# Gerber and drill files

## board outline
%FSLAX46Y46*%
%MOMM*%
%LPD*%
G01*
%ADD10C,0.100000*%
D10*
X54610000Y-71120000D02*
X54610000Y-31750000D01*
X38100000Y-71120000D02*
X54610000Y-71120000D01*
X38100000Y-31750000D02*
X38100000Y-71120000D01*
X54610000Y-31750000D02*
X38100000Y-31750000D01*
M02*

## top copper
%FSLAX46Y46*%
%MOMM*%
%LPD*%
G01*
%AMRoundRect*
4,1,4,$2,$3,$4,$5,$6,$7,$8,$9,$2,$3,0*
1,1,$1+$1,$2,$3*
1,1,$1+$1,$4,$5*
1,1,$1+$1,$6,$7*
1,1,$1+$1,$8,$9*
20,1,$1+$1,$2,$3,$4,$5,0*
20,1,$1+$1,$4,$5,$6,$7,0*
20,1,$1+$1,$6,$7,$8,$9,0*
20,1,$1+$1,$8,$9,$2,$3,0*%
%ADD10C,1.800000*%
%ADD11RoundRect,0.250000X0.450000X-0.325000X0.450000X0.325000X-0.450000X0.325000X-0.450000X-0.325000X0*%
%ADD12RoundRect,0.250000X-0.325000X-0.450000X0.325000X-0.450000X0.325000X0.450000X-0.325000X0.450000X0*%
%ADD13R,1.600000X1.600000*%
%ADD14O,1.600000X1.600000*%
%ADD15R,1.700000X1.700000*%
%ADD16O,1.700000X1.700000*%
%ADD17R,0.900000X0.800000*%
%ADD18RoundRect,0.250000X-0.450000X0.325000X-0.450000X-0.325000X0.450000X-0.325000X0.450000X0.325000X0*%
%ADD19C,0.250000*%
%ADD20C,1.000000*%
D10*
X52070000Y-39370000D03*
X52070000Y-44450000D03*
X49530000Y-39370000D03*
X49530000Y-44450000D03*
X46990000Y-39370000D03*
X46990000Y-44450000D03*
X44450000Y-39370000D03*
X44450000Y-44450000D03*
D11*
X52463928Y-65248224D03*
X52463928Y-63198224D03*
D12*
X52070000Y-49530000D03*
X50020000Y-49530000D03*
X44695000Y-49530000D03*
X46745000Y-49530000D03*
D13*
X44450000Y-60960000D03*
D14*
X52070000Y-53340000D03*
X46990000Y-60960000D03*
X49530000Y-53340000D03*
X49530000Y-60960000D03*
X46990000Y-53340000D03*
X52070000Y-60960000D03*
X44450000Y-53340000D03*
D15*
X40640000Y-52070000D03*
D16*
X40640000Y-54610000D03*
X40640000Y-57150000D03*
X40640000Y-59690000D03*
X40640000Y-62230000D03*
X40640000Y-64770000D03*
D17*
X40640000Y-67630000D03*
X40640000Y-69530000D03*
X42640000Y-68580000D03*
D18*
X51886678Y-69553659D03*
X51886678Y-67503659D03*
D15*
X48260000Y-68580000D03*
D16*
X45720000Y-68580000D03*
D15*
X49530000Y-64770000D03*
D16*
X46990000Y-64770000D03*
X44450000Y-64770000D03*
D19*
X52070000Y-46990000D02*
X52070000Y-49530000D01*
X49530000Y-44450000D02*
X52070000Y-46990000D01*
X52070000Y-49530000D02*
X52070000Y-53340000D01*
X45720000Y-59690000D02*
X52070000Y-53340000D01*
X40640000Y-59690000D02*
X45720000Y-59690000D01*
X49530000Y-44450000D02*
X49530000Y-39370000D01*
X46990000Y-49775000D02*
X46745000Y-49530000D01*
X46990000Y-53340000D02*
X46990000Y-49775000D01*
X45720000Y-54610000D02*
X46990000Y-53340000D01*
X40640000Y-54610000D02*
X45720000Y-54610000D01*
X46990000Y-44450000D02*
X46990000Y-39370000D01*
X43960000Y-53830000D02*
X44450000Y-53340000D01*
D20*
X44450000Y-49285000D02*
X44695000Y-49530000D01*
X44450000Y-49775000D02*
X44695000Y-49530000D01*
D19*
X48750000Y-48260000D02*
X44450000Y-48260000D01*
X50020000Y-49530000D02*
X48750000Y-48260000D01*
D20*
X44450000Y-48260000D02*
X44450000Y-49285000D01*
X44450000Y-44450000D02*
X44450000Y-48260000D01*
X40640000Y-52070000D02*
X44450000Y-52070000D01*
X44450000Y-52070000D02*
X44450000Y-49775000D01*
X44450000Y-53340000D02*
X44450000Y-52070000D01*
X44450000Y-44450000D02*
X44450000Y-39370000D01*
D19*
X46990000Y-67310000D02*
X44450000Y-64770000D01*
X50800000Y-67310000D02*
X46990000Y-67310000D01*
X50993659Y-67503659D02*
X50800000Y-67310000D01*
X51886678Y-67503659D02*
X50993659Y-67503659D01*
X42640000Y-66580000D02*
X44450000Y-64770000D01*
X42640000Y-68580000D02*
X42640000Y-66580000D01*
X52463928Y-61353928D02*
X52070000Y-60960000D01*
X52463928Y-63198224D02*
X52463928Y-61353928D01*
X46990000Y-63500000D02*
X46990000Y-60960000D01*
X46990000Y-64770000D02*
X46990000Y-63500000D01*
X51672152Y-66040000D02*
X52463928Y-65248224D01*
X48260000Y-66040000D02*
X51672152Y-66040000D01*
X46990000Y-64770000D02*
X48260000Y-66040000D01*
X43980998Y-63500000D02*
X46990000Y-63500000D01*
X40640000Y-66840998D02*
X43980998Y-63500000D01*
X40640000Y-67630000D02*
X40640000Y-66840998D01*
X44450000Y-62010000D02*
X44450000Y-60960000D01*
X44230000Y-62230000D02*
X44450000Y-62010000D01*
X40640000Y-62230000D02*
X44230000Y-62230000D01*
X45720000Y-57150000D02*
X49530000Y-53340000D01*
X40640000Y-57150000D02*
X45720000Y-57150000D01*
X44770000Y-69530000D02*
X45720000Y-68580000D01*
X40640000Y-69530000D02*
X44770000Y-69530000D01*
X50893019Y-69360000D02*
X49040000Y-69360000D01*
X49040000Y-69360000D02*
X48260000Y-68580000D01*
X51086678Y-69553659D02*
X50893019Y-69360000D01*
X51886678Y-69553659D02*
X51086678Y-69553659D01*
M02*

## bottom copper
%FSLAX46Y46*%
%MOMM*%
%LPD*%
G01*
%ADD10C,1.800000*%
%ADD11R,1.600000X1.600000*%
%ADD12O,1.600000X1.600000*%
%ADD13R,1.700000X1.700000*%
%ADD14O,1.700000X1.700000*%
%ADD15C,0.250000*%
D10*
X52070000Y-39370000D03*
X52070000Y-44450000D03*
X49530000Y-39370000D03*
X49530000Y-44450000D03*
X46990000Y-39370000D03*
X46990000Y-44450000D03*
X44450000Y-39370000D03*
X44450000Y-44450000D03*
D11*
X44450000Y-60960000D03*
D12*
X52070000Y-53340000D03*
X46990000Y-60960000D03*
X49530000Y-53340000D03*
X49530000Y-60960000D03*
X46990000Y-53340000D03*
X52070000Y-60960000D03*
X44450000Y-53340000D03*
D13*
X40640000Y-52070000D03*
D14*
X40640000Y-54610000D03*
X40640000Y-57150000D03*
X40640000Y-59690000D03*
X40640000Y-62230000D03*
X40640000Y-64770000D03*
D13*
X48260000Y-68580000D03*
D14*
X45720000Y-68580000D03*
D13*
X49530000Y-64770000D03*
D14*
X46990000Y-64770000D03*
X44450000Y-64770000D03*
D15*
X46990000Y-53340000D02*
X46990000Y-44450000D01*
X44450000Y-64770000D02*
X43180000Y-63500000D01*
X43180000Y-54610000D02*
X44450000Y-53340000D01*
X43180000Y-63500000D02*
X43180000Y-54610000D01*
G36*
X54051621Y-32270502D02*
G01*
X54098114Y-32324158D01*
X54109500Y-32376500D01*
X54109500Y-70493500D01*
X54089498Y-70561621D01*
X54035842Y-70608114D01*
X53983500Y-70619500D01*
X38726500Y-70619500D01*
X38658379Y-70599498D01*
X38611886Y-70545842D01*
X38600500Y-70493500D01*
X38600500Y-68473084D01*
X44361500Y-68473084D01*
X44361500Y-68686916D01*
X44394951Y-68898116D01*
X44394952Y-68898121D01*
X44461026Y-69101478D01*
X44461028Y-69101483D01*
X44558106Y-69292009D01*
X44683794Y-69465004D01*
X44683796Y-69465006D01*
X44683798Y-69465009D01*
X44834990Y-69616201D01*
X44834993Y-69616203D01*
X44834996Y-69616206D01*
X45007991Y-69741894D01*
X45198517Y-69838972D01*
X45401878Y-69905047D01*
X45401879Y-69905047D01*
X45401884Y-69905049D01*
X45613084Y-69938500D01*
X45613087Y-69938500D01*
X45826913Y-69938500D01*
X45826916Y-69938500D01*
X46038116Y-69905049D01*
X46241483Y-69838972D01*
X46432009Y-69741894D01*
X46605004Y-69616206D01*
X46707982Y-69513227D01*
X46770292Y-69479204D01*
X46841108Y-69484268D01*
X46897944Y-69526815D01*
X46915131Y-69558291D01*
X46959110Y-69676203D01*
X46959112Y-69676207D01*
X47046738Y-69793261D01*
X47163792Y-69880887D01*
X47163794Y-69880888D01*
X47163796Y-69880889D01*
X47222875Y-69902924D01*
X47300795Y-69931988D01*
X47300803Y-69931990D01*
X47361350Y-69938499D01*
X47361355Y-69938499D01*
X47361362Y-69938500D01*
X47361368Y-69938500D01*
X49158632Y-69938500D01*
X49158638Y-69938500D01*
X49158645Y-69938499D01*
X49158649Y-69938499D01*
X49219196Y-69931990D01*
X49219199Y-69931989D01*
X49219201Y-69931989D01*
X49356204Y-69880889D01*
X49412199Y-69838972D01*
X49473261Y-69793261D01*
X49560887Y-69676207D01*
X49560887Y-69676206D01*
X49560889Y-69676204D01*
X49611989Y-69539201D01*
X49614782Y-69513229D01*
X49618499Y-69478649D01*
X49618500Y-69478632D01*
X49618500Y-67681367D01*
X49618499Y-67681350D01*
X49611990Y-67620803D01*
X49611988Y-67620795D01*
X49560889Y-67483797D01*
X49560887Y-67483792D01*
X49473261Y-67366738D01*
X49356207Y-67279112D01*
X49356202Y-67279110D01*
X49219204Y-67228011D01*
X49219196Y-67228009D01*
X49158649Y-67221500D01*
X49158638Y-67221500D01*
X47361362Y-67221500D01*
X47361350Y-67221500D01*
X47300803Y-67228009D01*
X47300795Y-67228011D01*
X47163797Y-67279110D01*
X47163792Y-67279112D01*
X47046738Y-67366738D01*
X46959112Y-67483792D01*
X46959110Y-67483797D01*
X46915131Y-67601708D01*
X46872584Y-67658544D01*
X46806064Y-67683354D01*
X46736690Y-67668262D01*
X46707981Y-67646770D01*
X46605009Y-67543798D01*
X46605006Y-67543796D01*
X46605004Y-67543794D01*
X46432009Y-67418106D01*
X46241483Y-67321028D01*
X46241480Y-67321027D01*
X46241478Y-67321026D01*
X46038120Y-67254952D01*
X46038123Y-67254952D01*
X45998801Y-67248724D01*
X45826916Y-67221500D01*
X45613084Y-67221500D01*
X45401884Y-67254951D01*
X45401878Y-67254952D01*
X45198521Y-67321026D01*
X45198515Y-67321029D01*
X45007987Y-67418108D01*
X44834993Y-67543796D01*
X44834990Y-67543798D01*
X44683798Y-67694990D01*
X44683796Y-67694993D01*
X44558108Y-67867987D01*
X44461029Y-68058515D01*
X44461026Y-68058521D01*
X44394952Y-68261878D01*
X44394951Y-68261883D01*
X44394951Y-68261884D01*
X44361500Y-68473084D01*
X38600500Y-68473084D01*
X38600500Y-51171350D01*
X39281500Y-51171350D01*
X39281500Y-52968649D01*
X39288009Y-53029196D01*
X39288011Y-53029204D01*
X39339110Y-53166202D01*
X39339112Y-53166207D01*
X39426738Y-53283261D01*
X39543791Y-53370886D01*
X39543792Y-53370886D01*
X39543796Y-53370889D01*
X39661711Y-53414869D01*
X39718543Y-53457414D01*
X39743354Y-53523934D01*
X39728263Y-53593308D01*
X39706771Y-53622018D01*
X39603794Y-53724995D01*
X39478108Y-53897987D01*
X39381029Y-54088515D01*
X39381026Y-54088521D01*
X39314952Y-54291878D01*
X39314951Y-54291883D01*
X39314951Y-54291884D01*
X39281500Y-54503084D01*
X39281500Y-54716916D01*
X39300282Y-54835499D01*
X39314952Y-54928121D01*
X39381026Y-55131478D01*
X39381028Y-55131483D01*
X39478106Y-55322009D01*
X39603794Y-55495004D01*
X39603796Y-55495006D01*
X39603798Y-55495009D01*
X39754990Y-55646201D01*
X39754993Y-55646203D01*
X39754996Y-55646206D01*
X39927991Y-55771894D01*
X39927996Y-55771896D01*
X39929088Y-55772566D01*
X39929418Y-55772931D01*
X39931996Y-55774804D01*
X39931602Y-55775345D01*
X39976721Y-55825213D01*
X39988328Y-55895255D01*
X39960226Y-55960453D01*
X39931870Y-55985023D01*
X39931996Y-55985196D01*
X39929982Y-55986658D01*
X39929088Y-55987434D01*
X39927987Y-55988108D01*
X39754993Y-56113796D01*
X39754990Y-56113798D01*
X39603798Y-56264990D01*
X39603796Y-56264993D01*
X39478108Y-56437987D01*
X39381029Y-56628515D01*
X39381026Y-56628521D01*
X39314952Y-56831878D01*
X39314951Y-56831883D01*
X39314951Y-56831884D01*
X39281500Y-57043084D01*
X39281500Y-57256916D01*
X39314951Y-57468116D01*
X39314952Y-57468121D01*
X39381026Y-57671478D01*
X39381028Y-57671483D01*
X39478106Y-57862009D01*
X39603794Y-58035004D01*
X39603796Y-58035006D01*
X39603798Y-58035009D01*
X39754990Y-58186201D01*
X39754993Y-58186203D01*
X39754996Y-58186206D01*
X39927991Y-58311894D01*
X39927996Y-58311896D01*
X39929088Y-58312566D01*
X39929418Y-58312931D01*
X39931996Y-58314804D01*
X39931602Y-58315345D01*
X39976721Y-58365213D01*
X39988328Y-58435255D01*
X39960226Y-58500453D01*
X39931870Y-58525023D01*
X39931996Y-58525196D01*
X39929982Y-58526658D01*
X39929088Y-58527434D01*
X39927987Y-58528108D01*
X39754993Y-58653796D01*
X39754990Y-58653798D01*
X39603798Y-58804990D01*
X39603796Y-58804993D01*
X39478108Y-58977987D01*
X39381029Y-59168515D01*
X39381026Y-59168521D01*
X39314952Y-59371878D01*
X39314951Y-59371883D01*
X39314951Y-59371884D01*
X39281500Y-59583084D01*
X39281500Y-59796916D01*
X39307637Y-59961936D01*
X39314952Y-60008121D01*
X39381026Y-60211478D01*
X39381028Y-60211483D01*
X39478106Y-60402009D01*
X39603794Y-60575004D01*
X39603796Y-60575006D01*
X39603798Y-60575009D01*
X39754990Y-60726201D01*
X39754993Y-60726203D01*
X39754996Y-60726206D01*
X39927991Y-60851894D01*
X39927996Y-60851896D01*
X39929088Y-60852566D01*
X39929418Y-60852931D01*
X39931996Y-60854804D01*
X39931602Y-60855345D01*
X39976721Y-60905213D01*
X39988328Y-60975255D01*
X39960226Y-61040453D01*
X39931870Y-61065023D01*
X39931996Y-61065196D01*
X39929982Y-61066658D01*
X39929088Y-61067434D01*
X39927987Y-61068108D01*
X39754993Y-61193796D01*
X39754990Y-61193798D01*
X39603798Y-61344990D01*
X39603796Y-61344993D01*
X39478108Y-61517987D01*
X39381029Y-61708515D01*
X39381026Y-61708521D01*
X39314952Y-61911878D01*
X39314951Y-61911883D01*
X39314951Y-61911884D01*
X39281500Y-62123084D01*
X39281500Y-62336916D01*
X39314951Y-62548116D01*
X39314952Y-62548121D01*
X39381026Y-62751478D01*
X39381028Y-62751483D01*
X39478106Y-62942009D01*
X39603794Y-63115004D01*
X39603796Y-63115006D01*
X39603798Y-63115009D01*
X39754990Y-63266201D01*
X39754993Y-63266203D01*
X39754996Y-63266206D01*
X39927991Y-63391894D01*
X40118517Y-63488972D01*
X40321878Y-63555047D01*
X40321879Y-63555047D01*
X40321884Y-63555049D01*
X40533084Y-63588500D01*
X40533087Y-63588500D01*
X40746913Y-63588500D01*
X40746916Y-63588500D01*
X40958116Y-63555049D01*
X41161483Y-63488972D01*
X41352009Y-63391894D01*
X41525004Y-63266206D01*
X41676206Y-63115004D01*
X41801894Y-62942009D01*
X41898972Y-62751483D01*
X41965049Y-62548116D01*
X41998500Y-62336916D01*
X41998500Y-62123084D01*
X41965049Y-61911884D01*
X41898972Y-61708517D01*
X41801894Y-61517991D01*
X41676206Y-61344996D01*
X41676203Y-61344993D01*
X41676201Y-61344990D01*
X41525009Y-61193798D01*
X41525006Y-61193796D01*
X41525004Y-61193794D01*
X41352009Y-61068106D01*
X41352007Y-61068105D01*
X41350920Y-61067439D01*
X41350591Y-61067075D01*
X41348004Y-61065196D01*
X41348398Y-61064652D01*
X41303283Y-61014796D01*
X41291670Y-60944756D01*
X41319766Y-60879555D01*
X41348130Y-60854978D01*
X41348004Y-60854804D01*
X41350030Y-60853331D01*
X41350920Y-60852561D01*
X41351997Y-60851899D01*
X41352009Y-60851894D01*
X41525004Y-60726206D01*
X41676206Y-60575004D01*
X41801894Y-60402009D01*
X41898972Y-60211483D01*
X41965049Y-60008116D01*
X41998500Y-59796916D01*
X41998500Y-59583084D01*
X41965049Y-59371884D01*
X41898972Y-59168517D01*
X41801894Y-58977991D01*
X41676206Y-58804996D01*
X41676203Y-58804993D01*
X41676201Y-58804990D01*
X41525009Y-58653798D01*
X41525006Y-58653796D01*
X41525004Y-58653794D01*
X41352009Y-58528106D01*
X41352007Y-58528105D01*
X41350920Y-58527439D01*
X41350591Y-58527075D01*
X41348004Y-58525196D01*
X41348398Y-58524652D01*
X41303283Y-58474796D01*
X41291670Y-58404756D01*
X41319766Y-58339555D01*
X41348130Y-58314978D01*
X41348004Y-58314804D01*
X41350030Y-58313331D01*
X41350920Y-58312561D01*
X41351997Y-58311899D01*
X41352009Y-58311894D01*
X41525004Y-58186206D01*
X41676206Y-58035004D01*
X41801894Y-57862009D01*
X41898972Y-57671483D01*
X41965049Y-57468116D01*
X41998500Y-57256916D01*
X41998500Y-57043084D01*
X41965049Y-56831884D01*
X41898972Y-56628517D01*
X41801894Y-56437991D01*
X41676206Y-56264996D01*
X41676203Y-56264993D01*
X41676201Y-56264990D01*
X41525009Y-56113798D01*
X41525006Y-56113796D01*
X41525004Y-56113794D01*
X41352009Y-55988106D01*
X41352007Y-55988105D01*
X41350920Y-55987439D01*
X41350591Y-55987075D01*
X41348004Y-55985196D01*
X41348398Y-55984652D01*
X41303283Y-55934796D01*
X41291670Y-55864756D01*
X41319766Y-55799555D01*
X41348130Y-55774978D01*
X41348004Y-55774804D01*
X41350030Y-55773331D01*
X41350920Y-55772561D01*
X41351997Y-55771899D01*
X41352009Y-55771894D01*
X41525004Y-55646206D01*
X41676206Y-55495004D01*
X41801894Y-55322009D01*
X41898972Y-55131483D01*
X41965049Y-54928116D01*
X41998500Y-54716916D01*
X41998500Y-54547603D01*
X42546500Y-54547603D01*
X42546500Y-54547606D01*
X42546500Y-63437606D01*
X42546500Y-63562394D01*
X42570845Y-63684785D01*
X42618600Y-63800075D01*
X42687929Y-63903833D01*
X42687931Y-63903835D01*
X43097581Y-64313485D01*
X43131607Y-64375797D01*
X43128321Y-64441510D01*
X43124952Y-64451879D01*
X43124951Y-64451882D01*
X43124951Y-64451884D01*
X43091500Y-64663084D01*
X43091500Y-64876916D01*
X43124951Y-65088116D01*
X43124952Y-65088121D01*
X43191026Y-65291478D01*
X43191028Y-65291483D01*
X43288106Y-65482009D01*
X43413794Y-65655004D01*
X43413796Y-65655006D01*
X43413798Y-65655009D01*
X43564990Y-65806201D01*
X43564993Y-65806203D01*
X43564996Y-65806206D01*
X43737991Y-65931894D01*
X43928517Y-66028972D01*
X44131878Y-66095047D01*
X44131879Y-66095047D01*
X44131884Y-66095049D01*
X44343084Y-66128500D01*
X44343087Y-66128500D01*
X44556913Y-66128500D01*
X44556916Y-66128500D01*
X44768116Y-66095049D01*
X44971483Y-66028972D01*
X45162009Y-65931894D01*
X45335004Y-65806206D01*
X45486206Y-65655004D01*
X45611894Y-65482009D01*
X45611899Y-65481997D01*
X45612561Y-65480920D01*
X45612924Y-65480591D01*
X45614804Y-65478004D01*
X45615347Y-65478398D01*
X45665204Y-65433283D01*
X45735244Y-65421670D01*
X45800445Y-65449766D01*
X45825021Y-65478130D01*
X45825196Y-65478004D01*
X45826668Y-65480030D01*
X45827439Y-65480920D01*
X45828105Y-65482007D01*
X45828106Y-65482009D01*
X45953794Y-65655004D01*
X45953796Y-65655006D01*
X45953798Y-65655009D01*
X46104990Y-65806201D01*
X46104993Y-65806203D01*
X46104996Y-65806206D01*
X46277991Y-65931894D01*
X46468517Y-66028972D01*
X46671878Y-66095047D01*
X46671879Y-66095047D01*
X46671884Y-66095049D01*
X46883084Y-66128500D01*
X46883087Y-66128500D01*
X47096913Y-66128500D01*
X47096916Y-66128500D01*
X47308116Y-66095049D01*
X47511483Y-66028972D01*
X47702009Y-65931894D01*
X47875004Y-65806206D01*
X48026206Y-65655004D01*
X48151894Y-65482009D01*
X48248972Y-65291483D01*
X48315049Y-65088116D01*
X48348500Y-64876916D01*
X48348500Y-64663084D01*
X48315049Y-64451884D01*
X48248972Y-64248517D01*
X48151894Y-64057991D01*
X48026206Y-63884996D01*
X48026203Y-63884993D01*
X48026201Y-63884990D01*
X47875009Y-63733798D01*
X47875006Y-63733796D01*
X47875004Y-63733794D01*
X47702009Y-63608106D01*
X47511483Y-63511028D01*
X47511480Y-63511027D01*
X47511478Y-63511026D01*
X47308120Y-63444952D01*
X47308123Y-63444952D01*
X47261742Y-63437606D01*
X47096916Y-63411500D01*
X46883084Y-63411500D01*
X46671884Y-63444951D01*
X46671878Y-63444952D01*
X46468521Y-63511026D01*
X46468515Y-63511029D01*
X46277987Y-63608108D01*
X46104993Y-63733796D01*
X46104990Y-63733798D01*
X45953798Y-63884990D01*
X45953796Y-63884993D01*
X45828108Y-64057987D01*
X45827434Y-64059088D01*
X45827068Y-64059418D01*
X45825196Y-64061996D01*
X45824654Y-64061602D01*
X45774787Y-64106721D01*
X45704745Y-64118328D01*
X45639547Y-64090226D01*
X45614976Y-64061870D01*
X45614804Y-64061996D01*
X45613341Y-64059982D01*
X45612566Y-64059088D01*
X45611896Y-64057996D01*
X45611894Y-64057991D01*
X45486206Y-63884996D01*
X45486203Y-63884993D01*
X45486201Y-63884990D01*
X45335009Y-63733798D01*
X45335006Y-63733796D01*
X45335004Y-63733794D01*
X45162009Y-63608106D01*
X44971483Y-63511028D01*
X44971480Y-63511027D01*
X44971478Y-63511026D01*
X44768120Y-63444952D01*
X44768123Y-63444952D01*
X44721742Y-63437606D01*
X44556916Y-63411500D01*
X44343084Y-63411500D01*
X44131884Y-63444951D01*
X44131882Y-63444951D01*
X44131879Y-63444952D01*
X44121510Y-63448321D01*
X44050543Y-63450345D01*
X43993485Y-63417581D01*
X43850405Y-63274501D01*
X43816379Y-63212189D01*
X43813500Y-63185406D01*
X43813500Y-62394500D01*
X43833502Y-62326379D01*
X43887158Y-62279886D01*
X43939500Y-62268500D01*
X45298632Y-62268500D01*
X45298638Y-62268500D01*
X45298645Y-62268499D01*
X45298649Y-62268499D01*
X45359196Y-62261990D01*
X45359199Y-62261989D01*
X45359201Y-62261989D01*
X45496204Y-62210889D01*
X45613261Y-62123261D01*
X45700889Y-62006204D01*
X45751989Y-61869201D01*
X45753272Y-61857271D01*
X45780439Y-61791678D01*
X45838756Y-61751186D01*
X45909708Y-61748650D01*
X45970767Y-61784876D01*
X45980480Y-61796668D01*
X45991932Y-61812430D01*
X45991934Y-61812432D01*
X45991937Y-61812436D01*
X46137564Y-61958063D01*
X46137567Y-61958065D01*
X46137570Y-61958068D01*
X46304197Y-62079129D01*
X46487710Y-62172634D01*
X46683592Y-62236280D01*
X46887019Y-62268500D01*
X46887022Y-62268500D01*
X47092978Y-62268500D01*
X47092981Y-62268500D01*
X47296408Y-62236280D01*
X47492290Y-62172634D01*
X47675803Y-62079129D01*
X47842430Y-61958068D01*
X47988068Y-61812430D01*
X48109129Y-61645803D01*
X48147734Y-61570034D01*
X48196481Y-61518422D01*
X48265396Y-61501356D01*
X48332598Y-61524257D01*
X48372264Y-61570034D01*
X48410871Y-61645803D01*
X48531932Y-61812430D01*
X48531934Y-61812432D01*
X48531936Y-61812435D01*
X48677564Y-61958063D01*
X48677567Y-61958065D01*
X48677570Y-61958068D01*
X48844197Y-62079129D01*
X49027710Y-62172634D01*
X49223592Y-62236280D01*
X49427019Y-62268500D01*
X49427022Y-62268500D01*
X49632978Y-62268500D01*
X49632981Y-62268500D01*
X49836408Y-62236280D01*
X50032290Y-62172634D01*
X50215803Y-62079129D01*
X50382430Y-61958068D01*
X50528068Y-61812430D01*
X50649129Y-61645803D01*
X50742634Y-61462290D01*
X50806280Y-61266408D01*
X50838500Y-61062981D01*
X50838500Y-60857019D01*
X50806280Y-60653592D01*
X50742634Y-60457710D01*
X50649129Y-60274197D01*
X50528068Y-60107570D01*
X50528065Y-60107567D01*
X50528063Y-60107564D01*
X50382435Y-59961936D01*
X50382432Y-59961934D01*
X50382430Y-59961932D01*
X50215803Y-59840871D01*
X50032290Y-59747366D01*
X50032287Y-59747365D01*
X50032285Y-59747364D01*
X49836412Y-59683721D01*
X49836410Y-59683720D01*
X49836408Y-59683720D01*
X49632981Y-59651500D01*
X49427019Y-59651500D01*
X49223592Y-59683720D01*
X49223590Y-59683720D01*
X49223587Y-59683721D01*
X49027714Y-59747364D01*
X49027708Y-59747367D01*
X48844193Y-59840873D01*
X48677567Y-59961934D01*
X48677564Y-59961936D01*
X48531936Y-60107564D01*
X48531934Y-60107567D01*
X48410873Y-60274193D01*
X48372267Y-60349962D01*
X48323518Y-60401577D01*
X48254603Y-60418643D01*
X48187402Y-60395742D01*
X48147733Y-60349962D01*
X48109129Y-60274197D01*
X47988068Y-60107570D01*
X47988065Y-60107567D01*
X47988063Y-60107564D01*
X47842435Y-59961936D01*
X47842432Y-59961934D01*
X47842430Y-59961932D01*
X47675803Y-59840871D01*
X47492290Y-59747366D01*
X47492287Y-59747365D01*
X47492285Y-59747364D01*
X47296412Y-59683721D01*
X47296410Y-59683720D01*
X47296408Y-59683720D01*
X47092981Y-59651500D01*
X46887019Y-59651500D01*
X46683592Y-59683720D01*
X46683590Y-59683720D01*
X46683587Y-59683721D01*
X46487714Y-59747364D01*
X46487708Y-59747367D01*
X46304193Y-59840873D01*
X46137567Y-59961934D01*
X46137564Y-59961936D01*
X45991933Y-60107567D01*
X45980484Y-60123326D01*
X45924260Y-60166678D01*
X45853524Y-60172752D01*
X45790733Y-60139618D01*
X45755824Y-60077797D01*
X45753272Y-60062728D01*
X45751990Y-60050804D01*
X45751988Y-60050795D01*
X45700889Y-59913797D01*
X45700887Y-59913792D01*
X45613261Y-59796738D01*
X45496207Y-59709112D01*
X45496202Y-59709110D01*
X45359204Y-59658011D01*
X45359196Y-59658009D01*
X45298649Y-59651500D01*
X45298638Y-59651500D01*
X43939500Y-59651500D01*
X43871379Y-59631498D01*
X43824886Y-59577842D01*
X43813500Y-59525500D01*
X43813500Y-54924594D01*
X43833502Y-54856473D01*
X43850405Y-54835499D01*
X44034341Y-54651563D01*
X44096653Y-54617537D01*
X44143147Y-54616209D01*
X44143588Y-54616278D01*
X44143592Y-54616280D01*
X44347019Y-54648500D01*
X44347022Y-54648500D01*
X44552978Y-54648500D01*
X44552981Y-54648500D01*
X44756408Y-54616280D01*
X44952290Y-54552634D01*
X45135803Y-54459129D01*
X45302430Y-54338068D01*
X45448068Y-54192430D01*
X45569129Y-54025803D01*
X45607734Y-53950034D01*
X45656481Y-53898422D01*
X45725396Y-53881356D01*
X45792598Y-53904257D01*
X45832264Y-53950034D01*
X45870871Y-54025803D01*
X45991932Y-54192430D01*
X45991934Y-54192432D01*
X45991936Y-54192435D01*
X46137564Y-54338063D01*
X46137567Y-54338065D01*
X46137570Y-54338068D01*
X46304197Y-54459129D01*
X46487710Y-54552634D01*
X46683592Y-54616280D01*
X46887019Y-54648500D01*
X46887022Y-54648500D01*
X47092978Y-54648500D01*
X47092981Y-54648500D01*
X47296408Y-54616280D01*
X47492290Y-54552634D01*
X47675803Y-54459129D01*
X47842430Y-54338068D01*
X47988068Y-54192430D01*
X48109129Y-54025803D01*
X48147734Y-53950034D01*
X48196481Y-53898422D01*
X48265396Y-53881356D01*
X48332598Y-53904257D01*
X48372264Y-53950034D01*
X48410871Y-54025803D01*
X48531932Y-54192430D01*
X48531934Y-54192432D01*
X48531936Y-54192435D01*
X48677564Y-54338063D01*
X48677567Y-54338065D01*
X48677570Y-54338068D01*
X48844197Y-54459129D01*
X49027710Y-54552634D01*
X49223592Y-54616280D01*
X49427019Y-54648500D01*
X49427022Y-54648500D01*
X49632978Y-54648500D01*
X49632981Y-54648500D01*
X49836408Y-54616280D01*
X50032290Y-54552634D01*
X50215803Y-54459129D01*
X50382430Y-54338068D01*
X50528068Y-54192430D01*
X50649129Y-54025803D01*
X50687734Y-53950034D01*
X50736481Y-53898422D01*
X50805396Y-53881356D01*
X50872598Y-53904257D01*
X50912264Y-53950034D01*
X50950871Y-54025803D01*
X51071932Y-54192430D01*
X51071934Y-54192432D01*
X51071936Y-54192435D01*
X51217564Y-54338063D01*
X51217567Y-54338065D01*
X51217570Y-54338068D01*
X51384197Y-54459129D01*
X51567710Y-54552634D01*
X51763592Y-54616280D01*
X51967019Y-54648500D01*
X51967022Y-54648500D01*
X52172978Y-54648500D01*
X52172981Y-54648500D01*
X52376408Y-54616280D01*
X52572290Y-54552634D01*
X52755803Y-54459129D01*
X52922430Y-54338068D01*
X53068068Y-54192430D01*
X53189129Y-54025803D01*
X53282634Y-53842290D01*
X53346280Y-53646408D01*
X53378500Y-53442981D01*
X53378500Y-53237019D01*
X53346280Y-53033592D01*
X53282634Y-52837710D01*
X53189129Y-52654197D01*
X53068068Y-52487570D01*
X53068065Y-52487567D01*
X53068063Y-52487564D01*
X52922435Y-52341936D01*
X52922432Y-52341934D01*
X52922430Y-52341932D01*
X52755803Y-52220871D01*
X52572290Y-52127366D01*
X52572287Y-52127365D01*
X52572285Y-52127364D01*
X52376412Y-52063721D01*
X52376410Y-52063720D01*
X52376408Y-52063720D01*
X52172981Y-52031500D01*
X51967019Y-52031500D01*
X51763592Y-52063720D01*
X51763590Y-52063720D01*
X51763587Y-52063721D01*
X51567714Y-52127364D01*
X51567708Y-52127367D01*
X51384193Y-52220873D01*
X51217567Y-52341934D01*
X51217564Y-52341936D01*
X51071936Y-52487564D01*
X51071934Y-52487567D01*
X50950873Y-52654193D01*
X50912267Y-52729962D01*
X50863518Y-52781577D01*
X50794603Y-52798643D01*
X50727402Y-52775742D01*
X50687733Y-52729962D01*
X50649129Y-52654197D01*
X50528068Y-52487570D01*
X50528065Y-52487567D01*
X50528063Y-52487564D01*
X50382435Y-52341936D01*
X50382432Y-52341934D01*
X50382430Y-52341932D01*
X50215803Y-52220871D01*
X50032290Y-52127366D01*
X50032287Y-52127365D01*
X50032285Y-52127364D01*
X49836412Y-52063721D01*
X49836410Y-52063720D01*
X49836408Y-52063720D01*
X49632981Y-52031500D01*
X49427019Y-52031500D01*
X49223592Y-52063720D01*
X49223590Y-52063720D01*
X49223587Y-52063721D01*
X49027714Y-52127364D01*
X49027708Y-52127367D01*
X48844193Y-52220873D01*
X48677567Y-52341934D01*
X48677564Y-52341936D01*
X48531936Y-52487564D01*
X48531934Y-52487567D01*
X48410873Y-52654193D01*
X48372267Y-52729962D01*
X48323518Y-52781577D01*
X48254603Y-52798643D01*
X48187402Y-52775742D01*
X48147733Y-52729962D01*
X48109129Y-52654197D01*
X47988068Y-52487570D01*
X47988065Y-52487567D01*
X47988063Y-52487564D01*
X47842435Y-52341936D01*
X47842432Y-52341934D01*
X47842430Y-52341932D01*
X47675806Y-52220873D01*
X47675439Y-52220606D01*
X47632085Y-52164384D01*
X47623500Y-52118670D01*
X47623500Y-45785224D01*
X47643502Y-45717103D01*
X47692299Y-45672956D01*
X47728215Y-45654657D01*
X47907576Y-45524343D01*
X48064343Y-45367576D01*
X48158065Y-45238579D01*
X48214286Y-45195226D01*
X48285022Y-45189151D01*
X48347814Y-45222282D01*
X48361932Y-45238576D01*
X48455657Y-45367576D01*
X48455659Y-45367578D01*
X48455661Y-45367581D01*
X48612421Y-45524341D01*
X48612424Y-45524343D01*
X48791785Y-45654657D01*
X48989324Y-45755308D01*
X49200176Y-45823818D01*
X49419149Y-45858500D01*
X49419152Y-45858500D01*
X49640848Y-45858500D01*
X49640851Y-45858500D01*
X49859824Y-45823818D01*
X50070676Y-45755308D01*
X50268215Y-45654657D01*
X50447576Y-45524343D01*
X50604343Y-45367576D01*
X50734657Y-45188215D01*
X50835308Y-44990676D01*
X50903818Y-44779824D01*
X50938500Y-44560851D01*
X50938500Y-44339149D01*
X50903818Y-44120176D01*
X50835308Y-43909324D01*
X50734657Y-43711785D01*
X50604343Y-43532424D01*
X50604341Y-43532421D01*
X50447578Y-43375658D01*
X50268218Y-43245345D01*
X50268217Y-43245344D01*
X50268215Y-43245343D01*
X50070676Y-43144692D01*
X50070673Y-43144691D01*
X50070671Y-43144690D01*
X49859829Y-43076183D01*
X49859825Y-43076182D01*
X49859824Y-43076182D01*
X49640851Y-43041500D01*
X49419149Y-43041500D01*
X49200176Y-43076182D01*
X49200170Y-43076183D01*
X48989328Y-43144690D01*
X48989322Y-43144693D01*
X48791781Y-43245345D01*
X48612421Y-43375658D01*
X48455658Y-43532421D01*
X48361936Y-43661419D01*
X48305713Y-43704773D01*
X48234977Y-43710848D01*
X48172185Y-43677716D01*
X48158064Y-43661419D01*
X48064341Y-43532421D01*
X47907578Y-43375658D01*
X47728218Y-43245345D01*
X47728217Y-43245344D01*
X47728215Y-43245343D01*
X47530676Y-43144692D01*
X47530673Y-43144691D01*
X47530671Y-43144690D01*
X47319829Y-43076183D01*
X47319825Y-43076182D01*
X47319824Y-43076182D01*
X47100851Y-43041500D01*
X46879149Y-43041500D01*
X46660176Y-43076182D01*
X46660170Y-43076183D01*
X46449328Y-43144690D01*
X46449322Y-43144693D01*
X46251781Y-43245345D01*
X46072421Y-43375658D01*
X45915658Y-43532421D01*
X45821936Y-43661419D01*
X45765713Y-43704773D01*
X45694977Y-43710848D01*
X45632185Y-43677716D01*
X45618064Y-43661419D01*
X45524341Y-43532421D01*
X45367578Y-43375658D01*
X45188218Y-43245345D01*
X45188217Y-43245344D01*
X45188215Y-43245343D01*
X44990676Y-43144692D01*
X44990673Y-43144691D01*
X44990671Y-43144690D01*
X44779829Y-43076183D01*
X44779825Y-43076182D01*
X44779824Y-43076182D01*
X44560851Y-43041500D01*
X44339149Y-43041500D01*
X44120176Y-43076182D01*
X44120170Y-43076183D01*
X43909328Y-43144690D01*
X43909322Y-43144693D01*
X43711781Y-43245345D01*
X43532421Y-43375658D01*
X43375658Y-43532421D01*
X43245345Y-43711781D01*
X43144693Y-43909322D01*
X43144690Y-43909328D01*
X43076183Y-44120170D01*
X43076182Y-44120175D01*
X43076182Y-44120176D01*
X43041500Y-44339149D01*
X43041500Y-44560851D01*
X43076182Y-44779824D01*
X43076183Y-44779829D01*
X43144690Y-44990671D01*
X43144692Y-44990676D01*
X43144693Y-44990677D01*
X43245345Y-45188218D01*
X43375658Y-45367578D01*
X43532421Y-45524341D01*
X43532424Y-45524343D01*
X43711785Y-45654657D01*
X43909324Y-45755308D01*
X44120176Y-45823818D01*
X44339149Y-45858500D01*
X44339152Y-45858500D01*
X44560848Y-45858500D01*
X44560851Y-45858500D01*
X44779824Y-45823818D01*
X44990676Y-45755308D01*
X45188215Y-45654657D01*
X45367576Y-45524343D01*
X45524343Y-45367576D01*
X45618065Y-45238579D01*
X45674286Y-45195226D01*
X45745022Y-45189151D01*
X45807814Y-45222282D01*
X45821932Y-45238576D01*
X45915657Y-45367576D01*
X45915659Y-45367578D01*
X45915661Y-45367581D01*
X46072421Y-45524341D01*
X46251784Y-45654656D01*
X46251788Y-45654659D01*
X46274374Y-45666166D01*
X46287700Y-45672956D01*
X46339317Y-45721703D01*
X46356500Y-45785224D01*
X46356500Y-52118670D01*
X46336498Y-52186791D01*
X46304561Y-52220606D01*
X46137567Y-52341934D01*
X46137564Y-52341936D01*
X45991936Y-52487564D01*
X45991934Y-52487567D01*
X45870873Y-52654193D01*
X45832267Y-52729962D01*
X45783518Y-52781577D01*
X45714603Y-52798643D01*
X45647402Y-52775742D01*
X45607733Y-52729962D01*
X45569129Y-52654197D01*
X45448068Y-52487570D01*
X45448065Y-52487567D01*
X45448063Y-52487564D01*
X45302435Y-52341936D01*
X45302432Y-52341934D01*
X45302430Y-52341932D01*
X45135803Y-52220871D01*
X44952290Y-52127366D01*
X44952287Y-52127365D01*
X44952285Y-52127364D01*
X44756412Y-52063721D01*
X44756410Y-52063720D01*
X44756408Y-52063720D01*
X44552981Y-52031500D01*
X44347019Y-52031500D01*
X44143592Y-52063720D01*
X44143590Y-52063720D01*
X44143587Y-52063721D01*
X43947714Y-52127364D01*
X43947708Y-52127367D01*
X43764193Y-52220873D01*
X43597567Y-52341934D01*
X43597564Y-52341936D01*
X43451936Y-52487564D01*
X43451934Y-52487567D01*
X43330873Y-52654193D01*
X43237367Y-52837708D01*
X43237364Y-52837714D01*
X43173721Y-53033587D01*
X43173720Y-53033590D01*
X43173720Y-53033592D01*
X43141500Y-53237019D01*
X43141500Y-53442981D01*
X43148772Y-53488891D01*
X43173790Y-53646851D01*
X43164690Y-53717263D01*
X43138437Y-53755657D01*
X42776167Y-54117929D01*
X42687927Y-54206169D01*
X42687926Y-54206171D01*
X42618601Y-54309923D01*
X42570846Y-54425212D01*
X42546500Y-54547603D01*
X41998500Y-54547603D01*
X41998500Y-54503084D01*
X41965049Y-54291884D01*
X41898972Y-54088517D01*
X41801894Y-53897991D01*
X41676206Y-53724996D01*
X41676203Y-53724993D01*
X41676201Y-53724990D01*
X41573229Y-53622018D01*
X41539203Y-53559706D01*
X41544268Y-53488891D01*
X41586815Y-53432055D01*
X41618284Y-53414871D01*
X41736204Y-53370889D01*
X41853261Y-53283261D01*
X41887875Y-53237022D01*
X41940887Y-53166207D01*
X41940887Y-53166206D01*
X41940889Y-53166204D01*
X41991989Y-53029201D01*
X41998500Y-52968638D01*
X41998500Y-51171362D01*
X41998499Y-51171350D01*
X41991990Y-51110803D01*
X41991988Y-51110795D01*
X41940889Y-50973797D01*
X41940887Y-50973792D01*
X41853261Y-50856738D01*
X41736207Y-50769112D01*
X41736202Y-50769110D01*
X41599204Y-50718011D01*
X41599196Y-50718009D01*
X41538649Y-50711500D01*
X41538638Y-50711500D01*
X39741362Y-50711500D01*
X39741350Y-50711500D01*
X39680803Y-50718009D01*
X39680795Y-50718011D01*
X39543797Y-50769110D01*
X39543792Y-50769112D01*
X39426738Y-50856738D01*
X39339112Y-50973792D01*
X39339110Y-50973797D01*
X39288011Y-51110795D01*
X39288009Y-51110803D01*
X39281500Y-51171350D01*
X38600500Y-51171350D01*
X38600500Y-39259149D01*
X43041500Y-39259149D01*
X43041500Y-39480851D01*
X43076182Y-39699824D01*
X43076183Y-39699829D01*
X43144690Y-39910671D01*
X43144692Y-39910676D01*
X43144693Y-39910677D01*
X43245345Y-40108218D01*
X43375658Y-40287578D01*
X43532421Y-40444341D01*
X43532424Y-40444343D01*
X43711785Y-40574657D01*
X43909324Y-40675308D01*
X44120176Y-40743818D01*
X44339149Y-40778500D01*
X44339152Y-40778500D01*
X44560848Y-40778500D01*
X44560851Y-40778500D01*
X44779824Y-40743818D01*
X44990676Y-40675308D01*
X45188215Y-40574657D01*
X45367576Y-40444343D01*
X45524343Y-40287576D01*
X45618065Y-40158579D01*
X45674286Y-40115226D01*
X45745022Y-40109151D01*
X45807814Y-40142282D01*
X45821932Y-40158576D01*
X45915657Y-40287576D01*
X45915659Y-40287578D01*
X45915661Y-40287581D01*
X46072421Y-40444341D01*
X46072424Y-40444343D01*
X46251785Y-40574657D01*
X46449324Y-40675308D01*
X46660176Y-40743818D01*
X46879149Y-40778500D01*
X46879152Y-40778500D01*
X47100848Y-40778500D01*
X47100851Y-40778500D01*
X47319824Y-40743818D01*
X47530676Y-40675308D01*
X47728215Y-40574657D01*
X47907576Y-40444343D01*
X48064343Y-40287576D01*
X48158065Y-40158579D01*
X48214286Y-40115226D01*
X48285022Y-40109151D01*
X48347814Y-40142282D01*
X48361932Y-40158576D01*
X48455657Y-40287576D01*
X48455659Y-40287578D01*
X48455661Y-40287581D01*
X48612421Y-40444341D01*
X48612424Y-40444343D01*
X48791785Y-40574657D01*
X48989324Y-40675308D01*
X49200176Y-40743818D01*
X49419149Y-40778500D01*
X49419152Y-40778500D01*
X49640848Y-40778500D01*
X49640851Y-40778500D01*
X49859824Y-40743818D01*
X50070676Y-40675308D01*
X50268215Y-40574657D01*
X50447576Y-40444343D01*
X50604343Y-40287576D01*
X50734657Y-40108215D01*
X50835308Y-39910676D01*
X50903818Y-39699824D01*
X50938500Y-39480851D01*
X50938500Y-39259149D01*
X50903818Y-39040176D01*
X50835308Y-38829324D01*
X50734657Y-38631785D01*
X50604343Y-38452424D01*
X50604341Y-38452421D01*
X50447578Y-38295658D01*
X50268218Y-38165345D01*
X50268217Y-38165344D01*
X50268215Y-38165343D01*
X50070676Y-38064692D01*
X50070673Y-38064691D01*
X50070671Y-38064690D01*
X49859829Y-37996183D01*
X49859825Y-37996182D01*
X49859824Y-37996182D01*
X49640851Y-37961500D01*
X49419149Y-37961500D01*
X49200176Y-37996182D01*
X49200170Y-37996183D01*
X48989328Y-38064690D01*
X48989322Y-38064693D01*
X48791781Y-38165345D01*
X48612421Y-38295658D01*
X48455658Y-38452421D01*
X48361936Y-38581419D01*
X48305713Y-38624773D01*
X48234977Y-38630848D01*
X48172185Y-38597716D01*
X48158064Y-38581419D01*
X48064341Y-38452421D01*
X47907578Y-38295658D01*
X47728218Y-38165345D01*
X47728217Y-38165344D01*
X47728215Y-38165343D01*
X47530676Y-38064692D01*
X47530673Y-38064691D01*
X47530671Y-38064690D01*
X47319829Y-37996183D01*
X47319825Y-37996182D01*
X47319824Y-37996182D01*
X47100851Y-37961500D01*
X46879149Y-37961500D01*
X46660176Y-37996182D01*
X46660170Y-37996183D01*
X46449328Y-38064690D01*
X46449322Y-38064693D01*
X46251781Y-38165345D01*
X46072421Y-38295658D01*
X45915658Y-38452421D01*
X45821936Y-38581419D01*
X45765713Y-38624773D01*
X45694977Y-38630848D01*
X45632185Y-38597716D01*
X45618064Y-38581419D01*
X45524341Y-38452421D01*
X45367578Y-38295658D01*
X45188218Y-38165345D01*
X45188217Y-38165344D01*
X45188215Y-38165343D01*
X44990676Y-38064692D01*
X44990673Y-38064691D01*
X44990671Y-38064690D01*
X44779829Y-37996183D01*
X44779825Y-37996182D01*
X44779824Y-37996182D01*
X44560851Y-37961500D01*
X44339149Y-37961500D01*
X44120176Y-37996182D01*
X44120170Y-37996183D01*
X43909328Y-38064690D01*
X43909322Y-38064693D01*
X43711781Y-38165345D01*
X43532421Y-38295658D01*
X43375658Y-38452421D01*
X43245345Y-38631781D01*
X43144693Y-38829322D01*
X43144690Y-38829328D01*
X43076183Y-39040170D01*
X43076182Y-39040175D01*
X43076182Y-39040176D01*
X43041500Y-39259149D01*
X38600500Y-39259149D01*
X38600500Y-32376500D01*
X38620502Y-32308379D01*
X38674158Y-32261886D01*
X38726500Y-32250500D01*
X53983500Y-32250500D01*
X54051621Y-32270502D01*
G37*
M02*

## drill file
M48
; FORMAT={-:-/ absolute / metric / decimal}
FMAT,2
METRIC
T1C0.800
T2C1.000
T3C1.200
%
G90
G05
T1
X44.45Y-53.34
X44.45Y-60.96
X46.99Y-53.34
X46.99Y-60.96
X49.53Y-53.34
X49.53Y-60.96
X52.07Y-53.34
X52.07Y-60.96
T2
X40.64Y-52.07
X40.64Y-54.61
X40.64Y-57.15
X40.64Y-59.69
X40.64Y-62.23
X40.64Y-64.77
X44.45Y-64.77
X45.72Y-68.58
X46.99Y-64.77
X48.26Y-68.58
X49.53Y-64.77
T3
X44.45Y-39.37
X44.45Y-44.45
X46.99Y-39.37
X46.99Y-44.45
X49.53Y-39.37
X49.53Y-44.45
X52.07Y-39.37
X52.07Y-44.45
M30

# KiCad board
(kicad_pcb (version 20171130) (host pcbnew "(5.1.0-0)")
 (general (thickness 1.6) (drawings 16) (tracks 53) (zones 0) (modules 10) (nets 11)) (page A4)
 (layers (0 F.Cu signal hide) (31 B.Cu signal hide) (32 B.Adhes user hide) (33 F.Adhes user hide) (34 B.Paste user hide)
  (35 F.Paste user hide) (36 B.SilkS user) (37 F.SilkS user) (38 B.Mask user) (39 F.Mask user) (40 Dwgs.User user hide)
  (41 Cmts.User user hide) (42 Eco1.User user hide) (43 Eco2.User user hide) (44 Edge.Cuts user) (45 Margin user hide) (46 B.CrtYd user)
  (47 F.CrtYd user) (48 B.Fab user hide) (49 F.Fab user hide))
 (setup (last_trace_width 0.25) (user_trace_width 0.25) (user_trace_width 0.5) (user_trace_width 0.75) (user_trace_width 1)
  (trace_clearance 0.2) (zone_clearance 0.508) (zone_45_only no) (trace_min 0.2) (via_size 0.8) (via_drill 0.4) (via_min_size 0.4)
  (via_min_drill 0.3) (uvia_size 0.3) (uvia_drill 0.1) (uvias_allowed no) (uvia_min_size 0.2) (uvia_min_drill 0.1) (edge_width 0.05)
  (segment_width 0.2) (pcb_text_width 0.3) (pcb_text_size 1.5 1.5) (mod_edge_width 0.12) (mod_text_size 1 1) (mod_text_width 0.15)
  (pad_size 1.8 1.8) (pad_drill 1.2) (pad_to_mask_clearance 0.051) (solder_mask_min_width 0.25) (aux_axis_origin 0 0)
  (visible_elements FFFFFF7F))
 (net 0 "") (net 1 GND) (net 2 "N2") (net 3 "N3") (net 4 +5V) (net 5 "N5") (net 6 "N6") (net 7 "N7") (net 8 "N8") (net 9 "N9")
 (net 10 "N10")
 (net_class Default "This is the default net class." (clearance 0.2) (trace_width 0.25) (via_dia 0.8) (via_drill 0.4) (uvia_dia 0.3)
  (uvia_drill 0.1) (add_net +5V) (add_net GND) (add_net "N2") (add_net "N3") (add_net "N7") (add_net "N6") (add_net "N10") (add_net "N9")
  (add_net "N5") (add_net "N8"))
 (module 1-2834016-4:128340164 (layer F.Cu) (at 52.07 39.37 180)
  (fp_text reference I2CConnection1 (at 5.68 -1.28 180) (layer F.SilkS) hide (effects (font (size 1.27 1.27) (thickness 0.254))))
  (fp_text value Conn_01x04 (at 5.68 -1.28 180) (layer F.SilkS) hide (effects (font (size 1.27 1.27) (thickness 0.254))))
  (pad "" thru_hole circle (at 0 0 180) (size 1.8 1.8) (drill 1.2) (layers *.Cu *.Mask) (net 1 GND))
  (pad 1 thru_hole circle (at 0 -5.08 180) (size 1.8 1.8) (drill 1.2) (layers *.Cu *.Mask) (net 1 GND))
  (pad "" thru_hole circle (at 2.54 0 180) (size 1.8 1.8) (drill 1.2) (layers *.Cu *.Mask) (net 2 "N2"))
  (pad 2 thru_hole circle (at 2.54 -5.08 180) (size 1.8 1.8) (drill 1.2) (layers *.Cu *.Mask) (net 2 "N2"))
  (pad "" thru_hole circle (at 5.08 0 180) (size 1.8 1.8) (drill 1.2) (layers *.Cu *.Mask) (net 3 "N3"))
  (pad 3 thru_hole circle (at 5.08 -5.08 180) (size 1.8 1.8) (drill 1.2) (layers *.Cu *.Mask) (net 3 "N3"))
  (pad "" thru_hole circle (at 7.62 0 180) (size 1.8 1.8) (drill 1.2) (layers *.Cu *.Mask) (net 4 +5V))
  (pad 4 thru_hole circle (at 7.62 -5.08 180) (size 1.8 1.8) (drill 1.2) (layers *.Cu *.Mask) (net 4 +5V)))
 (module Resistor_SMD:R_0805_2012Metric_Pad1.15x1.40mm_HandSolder (layer F.Cu) (at 52.463928 64.223224 90)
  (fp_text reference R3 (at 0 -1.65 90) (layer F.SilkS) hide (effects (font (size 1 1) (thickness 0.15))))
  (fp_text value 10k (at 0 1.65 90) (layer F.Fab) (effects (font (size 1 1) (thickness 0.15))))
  (pad 1 smd roundrect (at -1.025 0 90) (size 1.15 1.4) (layers F.Cu F.Paste F.Mask) (roundrect_rratio 0.217391) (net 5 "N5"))
  (pad 2 smd roundrect (at 1.025 0 90) (size 1.15 1.4) (layers F.Cu F.Paste F.Mask) (roundrect_rratio 0.217391) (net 1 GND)))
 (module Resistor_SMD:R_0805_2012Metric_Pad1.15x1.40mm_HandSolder (layer F.Cu) (at 51.045 49.53)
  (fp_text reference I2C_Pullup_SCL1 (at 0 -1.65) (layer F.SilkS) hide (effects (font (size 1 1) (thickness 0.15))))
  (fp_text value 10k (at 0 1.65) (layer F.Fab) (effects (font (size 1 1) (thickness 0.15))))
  (pad 2 smd roundrect (at 1.025 0) (size 1.15 1.4) (layers F.Cu F.Paste F.Mask) (roundrect_rratio 0.217391) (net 2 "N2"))
  (pad 1 smd roundrect (at -1.025 0) (size 1.15 1.4) (layers F.Cu F.Paste F.Mask) (roundrect_rratio 0.217391) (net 4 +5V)))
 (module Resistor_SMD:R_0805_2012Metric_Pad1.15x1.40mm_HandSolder (layer F.Cu) (at 45.72 49.53)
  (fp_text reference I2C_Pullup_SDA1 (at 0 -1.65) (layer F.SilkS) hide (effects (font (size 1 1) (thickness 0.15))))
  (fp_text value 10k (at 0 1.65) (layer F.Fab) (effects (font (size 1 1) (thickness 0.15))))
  (pad 1 smd roundrect (at -1.025 0) (size 1.15 1.4) (layers F.Cu F.Paste F.Mask) (roundrect_rratio 0.217391) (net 4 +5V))
  (pad 2 smd roundrect (at 1.025 0) (size 1.15 1.4) (layers F.Cu F.Paste F.Mask) (roundrect_rratio 0.217391) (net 3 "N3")))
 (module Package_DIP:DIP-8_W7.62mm (layer F.Cu) (at 44.45 60.96 90)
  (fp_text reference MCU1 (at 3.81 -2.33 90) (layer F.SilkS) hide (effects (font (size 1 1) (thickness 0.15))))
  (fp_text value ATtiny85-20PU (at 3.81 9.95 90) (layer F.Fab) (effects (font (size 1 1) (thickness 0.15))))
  (pad 1 thru_hole rect (at 0 0 90) (size 1.6 1.6) (drill 0.8) (layers *.Cu *.Mask) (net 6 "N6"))
  (pad 5 thru_hole oval (at 7.62 7.62 90) (size 1.6 1.6) (drill 0.8) (layers *.Cu *.Mask) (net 2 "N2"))
  (pad 2 thru_hole oval (at 0 2.54 90) (size 1.6 1.6) (drill 0.8) (layers *.Cu *.Mask) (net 5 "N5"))
  (pad 6 thru_hole oval (at 7.62 5.08 90) (size 1.6 1.6) (drill 0.8) (layers *.Cu *.Mask) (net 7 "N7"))
  (pad 3 thru_hole oval (at 0 5.08 90) (size 1.6 1.6) (drill 0.8) (layers *.Cu *.Mask) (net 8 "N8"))
  (pad 7 thru_hole oval (at 7.62 2.54 90) (size 1.6 1.6) (drill 0.8) (layers *.Cu *.Mask) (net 3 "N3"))
  (pad 4 thru_hole oval (at 0 7.62 90) (size 1.6 1.6) (drill 0.8) (layers *.Cu *.Mask) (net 1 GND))
  (pad 8 thru_hole oval (at 7.62 0 90) (size 1.6 1.6) (drill 0.8) (layers *.Cu *.Mask) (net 4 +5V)))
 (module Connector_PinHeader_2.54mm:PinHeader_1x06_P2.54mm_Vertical (layer F.Cu) (at 40.64 52.07)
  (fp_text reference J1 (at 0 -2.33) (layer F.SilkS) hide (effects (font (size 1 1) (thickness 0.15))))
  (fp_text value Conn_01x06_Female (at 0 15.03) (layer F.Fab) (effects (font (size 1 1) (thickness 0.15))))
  (pad 1 thru_hole rect (at 0 0) (size 1.7 1.7) (drill 1) (layers *.Cu *.Mask) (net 4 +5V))
  (pad 2 thru_hole oval (at 0 2.54) (size 1.7 1.7) (drill 1) (layers *.Cu *.Mask) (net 3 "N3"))
  (pad 3 thru_hole oval (at 0 5.08) (size 1.7 1.7) (drill 1) (layers *.Cu *.Mask) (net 7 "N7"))
  (pad 4 thru_hole oval (at 0 7.62) (size 1.7 1.7) (drill 1) (layers *.Cu *.Mask) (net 2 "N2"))
  (pad 5 thru_hole oval (at 0 10.16) (size 1.7 1.7) (drill 1) (layers *.Cu *.Mask) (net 6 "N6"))
  (pad 6 thru_hole oval (at 0 12.7) (size 1.7 1.7) (drill 1) (layers *.Cu *.Mask) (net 1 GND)))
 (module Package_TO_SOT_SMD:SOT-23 (layer F.Cu) (at 41.64 68.58)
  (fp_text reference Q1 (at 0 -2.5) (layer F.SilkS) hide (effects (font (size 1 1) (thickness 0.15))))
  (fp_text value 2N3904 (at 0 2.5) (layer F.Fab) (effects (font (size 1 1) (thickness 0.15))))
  (pad 1 smd rect (at -1 -0.95) (size 0.9 0.8) (layers F.Cu F.Paste F.Mask) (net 5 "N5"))
  (pad 2 smd rect (at -1 0.95) (size 0.9 0.8) (layers F.Cu F.Paste F.Mask) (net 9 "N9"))
  (pad 3 smd rect (at 1 0) (size 0.9 0.8) (layers F.Cu F.Paste F.Mask) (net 4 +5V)))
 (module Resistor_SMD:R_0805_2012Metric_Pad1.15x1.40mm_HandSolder (layer F.Cu) (at 51.886678 68.528659 270)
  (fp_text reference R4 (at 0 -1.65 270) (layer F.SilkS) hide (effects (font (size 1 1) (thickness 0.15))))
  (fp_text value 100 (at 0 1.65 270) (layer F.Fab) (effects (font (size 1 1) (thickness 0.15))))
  (pad 2 smd roundrect (at 1.025 0 270) (size 1.15 1.4) (layers F.Cu F.Paste F.Mask) (roundrect_rratio 0.217391) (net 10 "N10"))
  (pad 1 smd roundrect (at -1.025 0 270) (size 1.15 1.4) (layers F.Cu F.Paste F.Mask) (roundrect_rratio 0.217391) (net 4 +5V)))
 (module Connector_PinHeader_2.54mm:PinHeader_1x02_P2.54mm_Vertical (layer F.Cu) (at 48.26 68.58 270)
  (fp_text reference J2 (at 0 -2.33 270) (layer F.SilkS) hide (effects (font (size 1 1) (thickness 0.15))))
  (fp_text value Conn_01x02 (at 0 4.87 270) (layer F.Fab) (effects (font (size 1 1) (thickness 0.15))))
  (pad 1 thru_hole rect (at 0 0 270) (size 1.7 1.7) (drill 1) (layers *.Cu *.Mask) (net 10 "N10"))
  (pad 2 thru_hole oval (at 0 2.54 270) (size 1.7 1.7) (drill 1) (layers *.Cu *.Mask) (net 9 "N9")))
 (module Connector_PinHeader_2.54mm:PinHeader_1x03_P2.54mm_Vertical (layer F.Cu) (at 49.53 64.77 270)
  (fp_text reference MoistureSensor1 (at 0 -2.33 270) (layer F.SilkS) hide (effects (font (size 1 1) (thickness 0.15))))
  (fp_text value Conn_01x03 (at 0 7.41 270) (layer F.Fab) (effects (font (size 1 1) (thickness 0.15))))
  (pad 1 thru_hole rect (at 0 0 270) (size 1.7 1.7) (drill 1) (layers *.Cu *.Mask) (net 1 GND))
  (pad 2 thru_hole oval (at 0 2.54 270) (size 1.7 1.7) (drill 1) (layers *.Cu *.Mask) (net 5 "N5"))
  (pad 3 thru_hole oval (at 0 5.08 270) (size 1.7 1.7) (drill 1) (layers *.Cu *.Mask) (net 4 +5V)))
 (gr_line (start 54.61 71.12) (end 54.61 31.75) (layer Edge.Cuts) (width 0.1))
 (gr_line (start 38.1 71.12) (end 54.61 71.12) (layer Edge.Cuts) (width 0.1))
 (gr_line (start 38.1 31.75) (end 38.1 71.12) (layer Edge.Cuts) (width 0.1))
 (gr_line (start 54.61 31.75) (end 38.1 31.75) (layer Edge.Cuts) (width 0.1))
 (segment (start 52.07 46.99) (end 52.07 49.53) (width 0.25) (layer F.Cu) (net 2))
 (segment (start 49.53 44.45) (end 52.07 46.99) (width 0.25) (layer F.Cu) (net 2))
 (segment (start 52.07 49.53) (end 52.07 53.34) (width 0.25) (layer F.Cu) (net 2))
 (segment (start 45.72 59.69) (end 52.07 53.34) (width 0.25) (layer F.Cu) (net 2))
 (segment (start 40.64 59.69) (end 45.72 59.69) (width 0.25) (layer F.Cu) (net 2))
 (segment (start 49.53 44.45) (end 49.53 39.37) (width 0.25) (layer F.Cu) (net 2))
 (segment (start 46.99 49.775) (end 46.745 49.53) (width 0.25) (layer F.Cu) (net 3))
 (segment (start 46.99 53.34) (end 46.99 49.775) (width 0.25) (layer F.Cu) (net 3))
 (segment (start 46.99 53.34) (end 46.99 44.45) (width 0.25) (layer B.Cu) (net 3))
 (segment (start 45.72 54.61) (end 46.99 53.34) (width 0.25) (layer F.Cu) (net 3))
 (segment (start 40.64 54.61) (end 45.72 54.61) (width 0.25) (layer F.Cu) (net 3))
 (segment (start 46.99 44.45) (end 46.99 39.37) (width 0.25) (layer F.Cu) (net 3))
 (segment (start 43.96 53.83) (end 44.45 53.34) (width 0.25) (layer F.Cu) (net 4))
 (segment (start 44.45 49.285) (end 44.695 49.53) (width 1) (layer F.Cu) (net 4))
 (segment (start 44.45 49.775) (end 44.695 49.53) (width 1) (layer F.Cu) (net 4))
 (segment (start 48.75 48.26) (end 44.45 48.26) (width 0.25) (layer F.Cu) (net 4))
 (segment (start 50.02 49.53) (end 48.75 48.26) (width 0.25) (layer F.Cu) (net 4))
 (segment (start 44.45 48.26) (end 44.45 49.285) (width 1) (layer F.Cu) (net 4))
 (segment (start 44.45 44.45) (end 44.45 48.26) (width 1) (layer F.Cu) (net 4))
 (segment (start 40.64 52.07) (end 44.45 52.07) (width 1) (layer F.Cu) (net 4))
 (segment (start 44.45 52.07) (end 44.45 49.775) (width 1) (layer F.Cu) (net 4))
 (segment (start 44.45 53.34) (end 44.45 52.07) (width 1) (layer F.Cu) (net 4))
 (segment (start 44.45 64.77) (end 43.18 63.5) (width 0.25) (layer B.Cu) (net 4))
 (segment (start 43.18 54.61) (end 44.45 53.34) (width 0.25) (layer B.Cu) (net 4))
 (segment (start 43.18 63.5) (end 43.18 54.61) (width 0.25) (layer B.Cu) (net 4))
 (segment (start 44.45 44.45) (end 44.45 39.37) (width 1) (layer F.Cu) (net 4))
 (segment (start 46.99 67.31) (end 44.45 64.77) (width 0.25) (layer F.Cu) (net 4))
 (segment (start 50.8 67.31) (end 46.99 67.31) (width 0.25) (layer F.Cu) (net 4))
 (segment (start 50.993659 67.503659) (end 50.8 67.31) (width 0.25) (layer F.Cu) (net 4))
 (segment (start 51.886678 67.503659) (end 50.993659 67.503659) (width 0.25) (layer F.Cu) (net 4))
 (segment (start 42.64 66.58) (end 44.45 64.77) (width 0.25) (layer F.Cu) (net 4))
 (segment (start 42.64 68.58) (end 42.64 66.58) (width 0.25) (layer F.Cu) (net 4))
 (segment (start 52.463928 61.353928) (end 52.07 60.96) (width 0.25) (layer F.Cu) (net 1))
 (segment (start 52.463928 63.198224) (end 52.463928 61.353928) (width 0.25) (layer F.Cu) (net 1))
 (segment (start 46.99 63.5) (end 46.99 60.96) (width 0.25) (layer F.Cu) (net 5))
 (segment (start 46.99 64.77) (end 46.99 63.5) (width 0.25) (layer F.Cu) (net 5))
 (segment (start 51.672152 66.04) (end 52.463928 65.248224) (width 0.25) (layer F.Cu) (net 5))
 (segment (start 48.26 66.04) (end 51.672152 66.04) (width 0.25) (layer F.Cu) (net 5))
 (segment (start 46.99 64.77) (end 48.26 66.04) (width 0.25) (layer F.Cu) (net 5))
 (segment (start 43.980998 63.5) (end 46.99 63.5) (width 0.25) (layer F.Cu) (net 5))
 (segment (start 40.64 66.840998) (end 43.980998 63.5) (width 0.25) (layer F.Cu) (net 5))
 (segment (start 40.64 67.63) (end 40.64 66.840998) (width 0.25) (layer F.Cu) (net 5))
 (segment (start 44.45 62.01) (end 44.45 60.96) (width 0.25) (layer F.Cu) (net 6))
 (segment (start 44.23 62.23) (end 44.45 62.01) (width 0.25) (layer F.Cu) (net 6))
 (segment (start 40.64 62.23) (end 44.23 62.23) (width 0.25) (layer F.Cu) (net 6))
 (segment (start 45.72 57.15) (end 49.53 53.34) (width 0.25) (layer F.Cu) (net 7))
 (segment (start 40.64 57.15) (end 45.72 57.15) (width 0.25) (layer F.Cu) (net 7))
 (segment (start 44.77 69.53) (end 45.72 68.58) (width 0.25) (layer F.Cu) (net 9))
 (segment (start 40.64 69.53) (end 44.77 69.53) (width 0.25) (layer F.Cu) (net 9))
 (segment (start 50.893019 69.36) (end 49.04 69.36) (width 0.25) (layer F.Cu) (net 10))
 (segment (start 49.04 69.36) (end 48.26 68.58) (width 0.25) (layer F.Cu) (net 10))
 (segment (start 51.086678 69.553659) (end 50.893019 69.36) (width 0.25) (layer F.Cu) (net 10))
 (segment (start 51.886678 69.553659) (end 51.086678 69.553659) (width 0.25) (layer F.Cu) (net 10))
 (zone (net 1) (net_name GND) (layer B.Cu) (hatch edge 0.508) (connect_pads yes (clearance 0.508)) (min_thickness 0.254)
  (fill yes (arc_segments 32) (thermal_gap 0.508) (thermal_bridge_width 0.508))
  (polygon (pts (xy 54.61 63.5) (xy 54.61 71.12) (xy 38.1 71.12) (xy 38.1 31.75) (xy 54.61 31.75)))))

